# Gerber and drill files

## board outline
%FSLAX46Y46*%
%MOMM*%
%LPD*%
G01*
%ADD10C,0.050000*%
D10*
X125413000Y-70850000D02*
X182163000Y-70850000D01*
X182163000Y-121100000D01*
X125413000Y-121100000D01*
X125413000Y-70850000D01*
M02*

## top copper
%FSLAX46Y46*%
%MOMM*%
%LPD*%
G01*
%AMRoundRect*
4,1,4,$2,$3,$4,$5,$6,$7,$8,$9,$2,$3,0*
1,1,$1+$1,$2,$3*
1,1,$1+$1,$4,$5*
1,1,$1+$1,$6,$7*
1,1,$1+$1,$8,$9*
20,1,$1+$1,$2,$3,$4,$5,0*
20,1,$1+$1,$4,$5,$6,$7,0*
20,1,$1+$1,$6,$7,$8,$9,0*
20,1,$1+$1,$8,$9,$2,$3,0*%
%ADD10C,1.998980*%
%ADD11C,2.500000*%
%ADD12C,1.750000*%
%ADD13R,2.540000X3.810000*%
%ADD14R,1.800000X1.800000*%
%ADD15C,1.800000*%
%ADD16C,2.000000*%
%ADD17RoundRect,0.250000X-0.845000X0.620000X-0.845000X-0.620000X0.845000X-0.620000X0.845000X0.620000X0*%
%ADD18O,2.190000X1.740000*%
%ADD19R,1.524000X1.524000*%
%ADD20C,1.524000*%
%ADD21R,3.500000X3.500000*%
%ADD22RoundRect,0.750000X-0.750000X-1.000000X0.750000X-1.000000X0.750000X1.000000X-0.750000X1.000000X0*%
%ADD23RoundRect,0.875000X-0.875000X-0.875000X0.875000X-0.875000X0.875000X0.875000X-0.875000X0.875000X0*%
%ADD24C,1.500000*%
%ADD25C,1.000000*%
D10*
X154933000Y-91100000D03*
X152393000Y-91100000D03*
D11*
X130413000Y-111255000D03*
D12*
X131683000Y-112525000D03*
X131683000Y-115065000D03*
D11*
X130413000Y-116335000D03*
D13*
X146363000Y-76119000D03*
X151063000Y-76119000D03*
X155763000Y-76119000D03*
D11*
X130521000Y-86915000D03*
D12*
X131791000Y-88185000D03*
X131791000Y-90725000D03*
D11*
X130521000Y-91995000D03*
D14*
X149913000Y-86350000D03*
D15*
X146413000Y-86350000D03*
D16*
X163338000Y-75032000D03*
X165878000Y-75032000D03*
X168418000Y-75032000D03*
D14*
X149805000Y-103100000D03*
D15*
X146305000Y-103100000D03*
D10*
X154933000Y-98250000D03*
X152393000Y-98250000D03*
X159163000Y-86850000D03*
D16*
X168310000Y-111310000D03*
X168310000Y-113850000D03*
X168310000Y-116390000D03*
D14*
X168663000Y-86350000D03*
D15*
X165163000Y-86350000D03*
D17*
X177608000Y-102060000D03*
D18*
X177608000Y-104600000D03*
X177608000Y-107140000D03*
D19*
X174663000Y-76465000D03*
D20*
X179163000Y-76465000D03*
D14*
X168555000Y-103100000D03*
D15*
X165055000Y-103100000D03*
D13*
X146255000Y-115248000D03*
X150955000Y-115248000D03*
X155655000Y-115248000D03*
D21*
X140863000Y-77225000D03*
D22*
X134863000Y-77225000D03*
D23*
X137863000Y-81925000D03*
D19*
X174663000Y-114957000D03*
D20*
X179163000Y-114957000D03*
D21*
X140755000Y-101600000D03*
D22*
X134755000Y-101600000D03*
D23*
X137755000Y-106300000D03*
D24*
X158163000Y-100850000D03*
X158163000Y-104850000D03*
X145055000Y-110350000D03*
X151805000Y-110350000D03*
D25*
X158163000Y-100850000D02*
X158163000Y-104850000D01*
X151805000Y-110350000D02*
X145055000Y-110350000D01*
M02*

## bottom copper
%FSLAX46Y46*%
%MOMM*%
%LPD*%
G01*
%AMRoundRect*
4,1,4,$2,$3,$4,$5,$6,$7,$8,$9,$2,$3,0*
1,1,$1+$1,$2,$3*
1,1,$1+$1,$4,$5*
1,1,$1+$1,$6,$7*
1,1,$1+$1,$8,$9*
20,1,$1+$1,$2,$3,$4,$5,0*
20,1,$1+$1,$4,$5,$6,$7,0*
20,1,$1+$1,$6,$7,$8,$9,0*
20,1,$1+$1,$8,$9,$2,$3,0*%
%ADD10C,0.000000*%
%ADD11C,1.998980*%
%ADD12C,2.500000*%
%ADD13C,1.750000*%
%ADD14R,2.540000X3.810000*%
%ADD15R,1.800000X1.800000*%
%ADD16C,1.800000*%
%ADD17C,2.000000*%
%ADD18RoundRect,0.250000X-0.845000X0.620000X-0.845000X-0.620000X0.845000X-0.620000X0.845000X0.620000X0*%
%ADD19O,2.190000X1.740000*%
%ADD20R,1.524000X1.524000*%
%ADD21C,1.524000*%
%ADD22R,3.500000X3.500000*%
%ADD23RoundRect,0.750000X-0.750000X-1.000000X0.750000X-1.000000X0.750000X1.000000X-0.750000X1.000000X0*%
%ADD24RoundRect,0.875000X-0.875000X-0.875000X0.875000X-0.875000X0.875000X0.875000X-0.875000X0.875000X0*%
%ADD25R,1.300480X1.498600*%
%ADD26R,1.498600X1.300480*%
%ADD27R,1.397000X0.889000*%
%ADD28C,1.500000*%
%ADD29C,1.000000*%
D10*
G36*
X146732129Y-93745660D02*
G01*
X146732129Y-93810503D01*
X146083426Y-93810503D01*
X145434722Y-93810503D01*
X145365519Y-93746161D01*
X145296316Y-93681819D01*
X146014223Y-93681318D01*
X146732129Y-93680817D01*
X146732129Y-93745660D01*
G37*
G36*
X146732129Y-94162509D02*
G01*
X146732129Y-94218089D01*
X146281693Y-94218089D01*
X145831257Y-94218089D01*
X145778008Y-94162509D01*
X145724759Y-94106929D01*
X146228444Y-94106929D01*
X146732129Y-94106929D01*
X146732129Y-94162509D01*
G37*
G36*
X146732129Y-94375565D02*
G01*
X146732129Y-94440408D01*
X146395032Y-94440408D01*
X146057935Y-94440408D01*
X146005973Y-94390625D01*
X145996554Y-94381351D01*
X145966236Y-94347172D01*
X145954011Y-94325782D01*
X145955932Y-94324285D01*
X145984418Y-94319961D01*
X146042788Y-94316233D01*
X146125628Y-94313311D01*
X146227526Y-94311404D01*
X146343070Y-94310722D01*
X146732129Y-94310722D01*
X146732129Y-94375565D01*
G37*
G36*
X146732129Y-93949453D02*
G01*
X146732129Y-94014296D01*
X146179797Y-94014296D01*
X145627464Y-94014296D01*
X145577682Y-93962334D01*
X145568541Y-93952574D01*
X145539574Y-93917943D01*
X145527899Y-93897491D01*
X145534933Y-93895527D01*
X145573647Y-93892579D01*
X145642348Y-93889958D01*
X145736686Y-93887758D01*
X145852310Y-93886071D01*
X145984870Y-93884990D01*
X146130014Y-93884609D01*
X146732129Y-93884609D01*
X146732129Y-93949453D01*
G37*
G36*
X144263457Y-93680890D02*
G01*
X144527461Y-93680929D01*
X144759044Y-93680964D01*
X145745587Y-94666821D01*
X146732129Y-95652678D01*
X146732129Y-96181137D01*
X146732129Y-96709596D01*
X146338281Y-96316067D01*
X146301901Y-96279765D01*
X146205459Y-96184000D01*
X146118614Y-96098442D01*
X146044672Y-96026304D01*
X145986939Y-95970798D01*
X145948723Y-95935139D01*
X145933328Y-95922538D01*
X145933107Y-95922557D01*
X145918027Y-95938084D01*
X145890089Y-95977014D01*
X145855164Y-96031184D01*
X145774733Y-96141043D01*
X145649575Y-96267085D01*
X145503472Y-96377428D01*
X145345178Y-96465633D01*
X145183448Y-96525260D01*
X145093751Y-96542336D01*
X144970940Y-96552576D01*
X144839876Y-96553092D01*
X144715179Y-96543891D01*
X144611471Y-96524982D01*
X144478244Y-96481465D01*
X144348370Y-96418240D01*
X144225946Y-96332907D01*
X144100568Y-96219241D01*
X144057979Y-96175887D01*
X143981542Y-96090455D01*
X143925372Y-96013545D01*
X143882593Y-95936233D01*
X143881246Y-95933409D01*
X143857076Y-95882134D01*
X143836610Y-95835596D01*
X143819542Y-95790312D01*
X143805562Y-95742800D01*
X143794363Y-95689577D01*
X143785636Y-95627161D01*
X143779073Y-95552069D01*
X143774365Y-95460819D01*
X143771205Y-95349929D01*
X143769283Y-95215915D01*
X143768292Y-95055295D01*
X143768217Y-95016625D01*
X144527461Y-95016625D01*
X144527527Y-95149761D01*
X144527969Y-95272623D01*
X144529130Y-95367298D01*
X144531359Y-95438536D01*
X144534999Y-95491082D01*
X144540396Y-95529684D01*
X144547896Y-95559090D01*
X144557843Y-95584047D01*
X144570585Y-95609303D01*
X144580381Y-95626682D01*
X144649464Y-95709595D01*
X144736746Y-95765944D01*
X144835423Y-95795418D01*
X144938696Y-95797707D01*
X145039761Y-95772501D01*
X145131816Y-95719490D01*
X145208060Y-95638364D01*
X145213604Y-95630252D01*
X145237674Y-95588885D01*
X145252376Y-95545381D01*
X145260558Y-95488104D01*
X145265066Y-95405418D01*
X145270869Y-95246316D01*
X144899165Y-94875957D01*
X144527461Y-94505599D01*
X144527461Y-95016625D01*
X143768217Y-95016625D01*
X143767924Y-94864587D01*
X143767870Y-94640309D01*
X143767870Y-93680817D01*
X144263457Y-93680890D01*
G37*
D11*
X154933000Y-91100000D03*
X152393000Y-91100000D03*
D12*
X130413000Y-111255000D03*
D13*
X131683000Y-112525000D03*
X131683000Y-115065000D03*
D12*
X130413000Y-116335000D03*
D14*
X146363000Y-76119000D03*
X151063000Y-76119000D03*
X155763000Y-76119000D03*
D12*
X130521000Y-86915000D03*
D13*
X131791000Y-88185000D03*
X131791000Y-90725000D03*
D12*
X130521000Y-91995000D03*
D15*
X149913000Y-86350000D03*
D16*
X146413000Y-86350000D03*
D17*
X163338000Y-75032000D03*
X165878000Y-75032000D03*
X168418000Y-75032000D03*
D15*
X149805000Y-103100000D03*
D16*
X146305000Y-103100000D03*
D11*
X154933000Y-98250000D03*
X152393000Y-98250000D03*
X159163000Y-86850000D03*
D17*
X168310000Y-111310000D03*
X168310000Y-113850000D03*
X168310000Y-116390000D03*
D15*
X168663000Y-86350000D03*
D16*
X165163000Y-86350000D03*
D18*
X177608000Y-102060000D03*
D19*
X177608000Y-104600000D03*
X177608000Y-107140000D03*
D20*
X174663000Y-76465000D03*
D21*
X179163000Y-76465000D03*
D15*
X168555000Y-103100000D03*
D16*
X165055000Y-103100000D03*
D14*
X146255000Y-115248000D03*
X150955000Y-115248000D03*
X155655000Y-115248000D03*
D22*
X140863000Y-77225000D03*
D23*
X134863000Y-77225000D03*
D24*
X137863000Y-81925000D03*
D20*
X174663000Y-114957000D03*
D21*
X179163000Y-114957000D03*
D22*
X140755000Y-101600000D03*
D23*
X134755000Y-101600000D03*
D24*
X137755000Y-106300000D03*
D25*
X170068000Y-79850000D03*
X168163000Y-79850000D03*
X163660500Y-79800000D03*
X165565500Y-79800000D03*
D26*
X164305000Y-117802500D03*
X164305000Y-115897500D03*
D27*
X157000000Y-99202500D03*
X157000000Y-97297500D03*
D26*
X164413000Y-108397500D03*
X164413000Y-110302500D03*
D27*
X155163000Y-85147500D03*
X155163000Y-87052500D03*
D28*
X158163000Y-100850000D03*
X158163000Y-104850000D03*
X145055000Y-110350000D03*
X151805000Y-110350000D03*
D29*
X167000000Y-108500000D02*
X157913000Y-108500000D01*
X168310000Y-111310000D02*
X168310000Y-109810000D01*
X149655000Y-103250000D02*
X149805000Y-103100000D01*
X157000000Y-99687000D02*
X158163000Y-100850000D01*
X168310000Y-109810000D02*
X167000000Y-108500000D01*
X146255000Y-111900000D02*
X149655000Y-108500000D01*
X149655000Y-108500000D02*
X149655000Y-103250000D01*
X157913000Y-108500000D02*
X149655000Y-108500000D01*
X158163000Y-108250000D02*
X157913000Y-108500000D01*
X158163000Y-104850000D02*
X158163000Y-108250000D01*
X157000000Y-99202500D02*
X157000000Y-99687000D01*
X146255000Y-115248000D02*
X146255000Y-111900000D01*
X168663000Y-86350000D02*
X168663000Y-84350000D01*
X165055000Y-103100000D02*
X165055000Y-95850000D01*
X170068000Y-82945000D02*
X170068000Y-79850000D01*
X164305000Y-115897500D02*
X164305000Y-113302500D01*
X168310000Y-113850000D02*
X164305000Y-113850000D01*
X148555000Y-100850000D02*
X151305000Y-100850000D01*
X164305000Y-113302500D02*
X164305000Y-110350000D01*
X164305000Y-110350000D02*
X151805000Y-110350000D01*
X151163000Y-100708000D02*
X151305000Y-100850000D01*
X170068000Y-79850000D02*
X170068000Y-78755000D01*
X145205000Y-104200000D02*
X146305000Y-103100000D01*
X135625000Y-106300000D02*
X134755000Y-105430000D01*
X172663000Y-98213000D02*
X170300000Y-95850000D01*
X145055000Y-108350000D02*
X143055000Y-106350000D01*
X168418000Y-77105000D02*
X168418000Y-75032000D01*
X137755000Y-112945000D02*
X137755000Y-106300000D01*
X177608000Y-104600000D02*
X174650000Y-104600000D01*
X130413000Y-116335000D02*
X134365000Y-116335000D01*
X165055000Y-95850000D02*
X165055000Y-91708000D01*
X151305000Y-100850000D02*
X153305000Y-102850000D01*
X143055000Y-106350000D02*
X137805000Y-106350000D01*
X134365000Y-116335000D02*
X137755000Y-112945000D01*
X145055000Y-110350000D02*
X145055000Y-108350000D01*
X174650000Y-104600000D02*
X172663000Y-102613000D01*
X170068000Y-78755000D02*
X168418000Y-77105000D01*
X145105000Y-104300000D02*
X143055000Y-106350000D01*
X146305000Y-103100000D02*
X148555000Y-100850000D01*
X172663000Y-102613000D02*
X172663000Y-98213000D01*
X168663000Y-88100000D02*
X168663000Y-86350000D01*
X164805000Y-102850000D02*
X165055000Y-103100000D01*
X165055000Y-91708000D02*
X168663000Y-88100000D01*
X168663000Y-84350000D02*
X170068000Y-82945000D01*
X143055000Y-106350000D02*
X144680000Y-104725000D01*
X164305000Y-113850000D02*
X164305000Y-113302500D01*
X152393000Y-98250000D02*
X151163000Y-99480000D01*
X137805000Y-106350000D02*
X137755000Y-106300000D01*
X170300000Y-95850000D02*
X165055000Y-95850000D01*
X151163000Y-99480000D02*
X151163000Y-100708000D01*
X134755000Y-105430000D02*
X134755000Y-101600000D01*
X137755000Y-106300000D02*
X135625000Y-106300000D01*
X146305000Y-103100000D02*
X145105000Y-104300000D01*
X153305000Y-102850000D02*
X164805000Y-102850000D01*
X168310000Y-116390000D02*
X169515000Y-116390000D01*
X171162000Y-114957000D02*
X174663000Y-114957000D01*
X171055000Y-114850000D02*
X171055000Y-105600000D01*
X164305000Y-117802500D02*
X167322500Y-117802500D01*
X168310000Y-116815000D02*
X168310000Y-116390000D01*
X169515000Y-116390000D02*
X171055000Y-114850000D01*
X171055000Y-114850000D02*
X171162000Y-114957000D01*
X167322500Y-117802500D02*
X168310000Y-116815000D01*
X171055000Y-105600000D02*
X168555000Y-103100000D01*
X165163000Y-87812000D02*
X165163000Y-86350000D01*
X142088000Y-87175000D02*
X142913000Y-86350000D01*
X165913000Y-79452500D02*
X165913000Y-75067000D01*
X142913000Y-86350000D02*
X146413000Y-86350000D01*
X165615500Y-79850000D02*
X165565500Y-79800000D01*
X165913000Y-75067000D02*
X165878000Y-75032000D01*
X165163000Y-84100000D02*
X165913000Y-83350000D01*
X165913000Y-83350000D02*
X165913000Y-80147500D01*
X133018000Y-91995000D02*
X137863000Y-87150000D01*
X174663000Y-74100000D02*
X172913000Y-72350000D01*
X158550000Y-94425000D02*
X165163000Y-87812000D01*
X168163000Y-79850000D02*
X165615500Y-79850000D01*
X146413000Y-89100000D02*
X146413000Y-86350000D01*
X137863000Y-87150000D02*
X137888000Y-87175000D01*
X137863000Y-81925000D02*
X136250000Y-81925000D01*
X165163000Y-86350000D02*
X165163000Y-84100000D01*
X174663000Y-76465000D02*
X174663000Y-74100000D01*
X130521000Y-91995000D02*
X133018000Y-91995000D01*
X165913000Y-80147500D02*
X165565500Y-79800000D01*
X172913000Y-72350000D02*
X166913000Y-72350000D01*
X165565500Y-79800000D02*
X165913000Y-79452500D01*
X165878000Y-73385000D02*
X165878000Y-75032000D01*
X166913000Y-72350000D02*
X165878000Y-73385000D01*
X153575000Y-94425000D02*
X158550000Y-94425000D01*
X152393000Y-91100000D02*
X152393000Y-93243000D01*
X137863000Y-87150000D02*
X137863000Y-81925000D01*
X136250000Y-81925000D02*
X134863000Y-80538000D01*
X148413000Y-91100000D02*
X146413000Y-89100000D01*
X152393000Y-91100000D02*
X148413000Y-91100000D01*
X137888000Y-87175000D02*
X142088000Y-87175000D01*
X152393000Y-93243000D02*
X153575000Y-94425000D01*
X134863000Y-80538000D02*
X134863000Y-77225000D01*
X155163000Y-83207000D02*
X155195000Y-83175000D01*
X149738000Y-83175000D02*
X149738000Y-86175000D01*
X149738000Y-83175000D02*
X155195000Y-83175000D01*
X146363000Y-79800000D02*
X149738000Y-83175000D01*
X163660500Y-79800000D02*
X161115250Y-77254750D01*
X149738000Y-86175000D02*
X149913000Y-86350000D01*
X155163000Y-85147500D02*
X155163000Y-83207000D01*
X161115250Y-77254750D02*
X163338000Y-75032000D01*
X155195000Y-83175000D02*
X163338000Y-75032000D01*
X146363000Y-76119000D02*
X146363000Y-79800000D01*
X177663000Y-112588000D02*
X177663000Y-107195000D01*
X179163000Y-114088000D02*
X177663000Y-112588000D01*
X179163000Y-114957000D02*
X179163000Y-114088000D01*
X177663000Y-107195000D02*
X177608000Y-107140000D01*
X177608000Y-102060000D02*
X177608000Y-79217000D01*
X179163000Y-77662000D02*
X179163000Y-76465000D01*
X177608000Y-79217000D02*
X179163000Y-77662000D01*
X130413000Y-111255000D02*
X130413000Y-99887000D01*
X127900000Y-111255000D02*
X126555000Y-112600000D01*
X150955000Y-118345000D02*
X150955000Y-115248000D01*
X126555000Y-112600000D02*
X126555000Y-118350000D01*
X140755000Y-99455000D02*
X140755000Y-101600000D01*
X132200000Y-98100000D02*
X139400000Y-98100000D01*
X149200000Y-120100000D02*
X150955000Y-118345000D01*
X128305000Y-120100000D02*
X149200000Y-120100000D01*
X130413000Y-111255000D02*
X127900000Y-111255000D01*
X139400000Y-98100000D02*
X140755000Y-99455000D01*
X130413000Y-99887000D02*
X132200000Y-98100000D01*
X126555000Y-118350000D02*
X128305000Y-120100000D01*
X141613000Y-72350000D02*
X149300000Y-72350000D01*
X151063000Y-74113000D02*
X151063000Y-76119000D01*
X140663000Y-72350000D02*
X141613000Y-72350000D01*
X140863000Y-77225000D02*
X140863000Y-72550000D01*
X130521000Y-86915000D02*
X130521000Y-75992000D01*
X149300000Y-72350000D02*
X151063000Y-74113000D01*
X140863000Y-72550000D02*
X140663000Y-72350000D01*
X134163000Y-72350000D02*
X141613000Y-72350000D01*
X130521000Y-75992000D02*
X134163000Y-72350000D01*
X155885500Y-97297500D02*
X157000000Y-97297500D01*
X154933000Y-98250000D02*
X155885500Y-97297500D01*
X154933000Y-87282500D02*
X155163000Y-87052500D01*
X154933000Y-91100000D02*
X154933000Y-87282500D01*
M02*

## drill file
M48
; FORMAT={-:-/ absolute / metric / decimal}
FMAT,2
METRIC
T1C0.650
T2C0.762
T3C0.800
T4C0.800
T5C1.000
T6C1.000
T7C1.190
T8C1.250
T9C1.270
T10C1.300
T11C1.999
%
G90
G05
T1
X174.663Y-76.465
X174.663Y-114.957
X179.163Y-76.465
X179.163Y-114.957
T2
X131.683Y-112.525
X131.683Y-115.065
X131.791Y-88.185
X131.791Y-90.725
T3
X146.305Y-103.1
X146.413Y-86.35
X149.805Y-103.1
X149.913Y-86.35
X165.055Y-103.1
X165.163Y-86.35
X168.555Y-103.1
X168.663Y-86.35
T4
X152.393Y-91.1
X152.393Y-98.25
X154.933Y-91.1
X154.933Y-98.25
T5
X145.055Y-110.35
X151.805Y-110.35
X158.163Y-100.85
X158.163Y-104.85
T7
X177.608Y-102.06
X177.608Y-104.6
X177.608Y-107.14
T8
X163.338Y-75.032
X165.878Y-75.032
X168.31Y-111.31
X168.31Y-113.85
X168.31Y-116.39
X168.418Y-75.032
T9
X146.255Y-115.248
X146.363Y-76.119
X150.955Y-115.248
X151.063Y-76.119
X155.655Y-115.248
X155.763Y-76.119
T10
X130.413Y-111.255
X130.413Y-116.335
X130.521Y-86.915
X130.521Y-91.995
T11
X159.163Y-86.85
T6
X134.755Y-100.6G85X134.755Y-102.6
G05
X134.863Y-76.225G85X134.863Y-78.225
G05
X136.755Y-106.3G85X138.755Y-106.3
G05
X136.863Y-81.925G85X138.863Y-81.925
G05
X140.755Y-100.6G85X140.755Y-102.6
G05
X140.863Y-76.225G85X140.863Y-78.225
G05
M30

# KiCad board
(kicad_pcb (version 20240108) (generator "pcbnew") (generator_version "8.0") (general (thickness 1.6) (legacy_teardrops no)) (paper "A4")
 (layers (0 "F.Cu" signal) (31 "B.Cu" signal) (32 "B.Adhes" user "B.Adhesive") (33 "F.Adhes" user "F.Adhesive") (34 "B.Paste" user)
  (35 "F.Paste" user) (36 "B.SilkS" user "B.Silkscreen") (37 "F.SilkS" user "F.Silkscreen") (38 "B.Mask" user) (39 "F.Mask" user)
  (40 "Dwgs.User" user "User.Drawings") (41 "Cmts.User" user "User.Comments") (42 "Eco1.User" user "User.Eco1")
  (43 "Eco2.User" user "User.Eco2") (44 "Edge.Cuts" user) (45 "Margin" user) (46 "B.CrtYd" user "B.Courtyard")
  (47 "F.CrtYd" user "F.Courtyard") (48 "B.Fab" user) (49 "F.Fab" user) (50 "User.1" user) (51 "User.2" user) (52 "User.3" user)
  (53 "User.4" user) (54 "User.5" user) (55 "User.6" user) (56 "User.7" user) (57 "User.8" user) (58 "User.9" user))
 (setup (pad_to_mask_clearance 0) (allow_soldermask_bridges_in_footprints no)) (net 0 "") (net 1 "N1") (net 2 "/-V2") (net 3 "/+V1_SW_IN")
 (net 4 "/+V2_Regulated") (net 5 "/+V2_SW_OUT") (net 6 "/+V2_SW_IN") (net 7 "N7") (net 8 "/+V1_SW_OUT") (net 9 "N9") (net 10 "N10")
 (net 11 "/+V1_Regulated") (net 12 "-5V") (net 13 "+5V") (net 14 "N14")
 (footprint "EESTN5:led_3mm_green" (layer "F.Cu") (at 153.663 91.1 -90)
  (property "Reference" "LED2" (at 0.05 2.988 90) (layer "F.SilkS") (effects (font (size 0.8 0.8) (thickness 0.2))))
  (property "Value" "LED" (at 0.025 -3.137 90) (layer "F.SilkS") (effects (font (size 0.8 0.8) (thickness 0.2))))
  (pad "1" thru_hole circle (at 0 -1.27 270) (size 1.99898 1.99898) (drill 0.8001) (layers "*.Cu" "*.Mask" "F.SilkS")
   (remove_unused_layers no) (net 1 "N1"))
  (pad "2" thru_hole circle (at 0 1.27 270) (size 1.99898 1.99898) (drill 0.8001) (layers "*.Cu" "*.Mask" "F.SilkS")
   (remove_unused_layers no) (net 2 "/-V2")))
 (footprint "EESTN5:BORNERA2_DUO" (layer "F.Cu") (at 130.413 113.795 -90)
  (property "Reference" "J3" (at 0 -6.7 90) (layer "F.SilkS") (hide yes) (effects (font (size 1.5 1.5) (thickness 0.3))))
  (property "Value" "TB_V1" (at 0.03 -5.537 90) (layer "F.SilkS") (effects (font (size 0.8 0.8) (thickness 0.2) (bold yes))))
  (pad "1" thru_hole circle (at -2.54 0 270) (size 2.5 2.5) (drill 1.3) (layers "*.Cu" "*.Mask" "F.SilkS") (remove_unused_layers no)
   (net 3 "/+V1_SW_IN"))
  (pad "1" thru_hole circle (at -1.27 -1.27 270) (size 1.75 1.75) (drill 0.762) (layers "*.Cu" "*.Mask") (remove_unused_layers no)
   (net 3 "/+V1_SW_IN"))
  (pad "2" thru_hole circle (at 1.27 -1.27 270) (size 1.75 1.75) (drill 0.762) (layers "*.Cu" "*.Mask") (remove_unused_layers no)
   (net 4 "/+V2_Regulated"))
  (pad "2" thru_hole circle (at 2.54 0 270) (size 2.5 2.5) (drill 1.3) (layers "*.Cu" "*.Mask" "F.SilkS") (remove_unused_layers no)
   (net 4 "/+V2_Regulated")))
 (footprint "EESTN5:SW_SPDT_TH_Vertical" (layer "F.Cu") (at 151.063 76.119 90)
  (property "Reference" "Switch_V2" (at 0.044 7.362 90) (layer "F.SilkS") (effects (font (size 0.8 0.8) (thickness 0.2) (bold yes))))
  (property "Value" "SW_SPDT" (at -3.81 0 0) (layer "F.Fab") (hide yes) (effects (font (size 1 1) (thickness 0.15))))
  (pad "1" thru_hole rect (at 0 -4.7 90) (size 3.81 2.54) (drill 1.27) (layers "*.Cu" "*.Mask") (remove_unused_layers no)
   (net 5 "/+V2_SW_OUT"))
  (pad "2" thru_hole rect (at 0 0 90) (size 3.81 2.54) (drill 1.27) (layers "*.Cu" "*.Mask") (remove_unused_layers no) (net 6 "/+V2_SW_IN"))
  (pad "3" thru_hole rect (at 0 4.7 90) (size 3.81 2.54) (drill 1.27) (layers "*.Cu" "*.Mask") (remove_unused_layers no) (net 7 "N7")))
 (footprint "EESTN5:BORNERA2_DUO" (layer "F.Cu") (at 130.521 89.455 -90)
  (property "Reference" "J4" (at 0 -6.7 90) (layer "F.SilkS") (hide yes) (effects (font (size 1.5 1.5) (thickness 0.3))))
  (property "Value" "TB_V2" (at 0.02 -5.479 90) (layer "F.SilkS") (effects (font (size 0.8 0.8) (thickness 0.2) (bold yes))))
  (pad "1" thru_hole circle (at -2.54 0 270) (size 2.5 2.5) (drill 1.3) (layers "*.Cu" "*.Mask" "F.SilkS") (remove_unused_layers no)
   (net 6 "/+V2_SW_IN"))
  (pad "1" thru_hole circle (at -1.27 -1.27 270) (size 1.75 1.75) (drill 0.762) (layers "*.Cu" "*.Mask") (remove_unused_layers no)
   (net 6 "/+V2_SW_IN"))
  (pad "2" thru_hole circle (at 1.27 -1.27 270) (size 1.75 1.75) (drill 0.762) (layers "*.Cu" "*.Mask") (remove_unused_layers no)
   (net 2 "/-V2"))
  (pad "2" thru_hole circle (at 2.54 0 270) (size 2.5 2.5) (drill 1.3) (layers "*.Cu" "*.Mask" "F.SilkS") (remove_unused_layers no)
   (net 2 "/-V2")))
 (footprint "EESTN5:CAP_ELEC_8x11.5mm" (layer "F.Cu") (at 148.163 86.35 90)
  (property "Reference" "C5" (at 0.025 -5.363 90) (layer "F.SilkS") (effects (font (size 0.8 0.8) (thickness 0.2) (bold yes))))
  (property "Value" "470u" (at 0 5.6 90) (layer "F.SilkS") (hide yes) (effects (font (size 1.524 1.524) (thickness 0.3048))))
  (pad "1" thru_hole rect (at 0 1.75 90) (size 1.8 1.8) (drill 0.8) (layers "*.Cu" "*.Mask" "F.SilkS") (remove_unused_layers no)
   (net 5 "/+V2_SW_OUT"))
  (pad "2" thru_hole circle (at 0 -1.75 90) (size 1.8 1.8) (drill 0.8) (layers "*.Cu" "*.Mask" "F.SilkS") (remove_unused_layers no)
   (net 2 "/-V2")))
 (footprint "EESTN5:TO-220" (layer "F.Cu") (at 165.878 75.032)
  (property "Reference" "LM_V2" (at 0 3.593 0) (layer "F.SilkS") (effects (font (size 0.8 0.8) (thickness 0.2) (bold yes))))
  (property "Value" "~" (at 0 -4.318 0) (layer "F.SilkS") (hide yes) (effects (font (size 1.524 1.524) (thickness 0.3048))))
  (pad "1" thru_hole circle (at -2.54 0) (size 2 2) (drill 1.24968) (layers "*.Cu" "*.Mask" "F.SilkS") (remove_unused_layers no)
   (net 5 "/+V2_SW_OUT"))
  (pad "2" thru_hole circle (at 0 0) (size 2 2) (drill 1.24968) (layers "*.Cu" "*.Mask" "F.SilkS") (remove_unused_layers no) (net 2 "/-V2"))
  (pad "3" thru_hole circle (at 2.54 0) (size 2 2) (drill 1.24968) (layers "*.Cu" "*.Mask" "F.SilkS") (remove_unused_layers no)
   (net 4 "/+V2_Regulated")))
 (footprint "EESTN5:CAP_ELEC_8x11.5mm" (layer "F.Cu") (at 148.055 103.1 90)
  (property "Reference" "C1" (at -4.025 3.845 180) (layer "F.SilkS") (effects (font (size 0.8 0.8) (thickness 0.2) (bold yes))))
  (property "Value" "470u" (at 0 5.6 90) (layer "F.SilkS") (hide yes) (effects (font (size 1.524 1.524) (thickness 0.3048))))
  (pad "1" thru_hole rect (at 0 1.75 90) (size 1.8 1.8) (drill 0.8) (layers "*.Cu" "*.Mask" "F.SilkS") (remove_unused_layers no)
   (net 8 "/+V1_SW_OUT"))
  (pad "2" thru_hole circle (at 0 -1.75 90) (size 1.8 1.8) (drill 0.8) (layers "*.Cu" "*.Mask" "F.SilkS") (remove_unused_layers no)
   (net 4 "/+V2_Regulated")))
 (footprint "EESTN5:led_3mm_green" (layer "F.Cu") (at 153.663 98.25 -90)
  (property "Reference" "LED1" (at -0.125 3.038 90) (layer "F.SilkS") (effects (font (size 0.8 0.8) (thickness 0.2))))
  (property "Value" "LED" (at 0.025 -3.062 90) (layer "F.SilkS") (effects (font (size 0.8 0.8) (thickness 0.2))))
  (pad "1" thru_hole circle (at 0 -1.27 270) (size 1.99898 1.99898) (drill 0.8001) (layers "*.Cu" "*.Mask" "F.SilkS")
   (remove_unused_layers no) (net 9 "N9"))
  (pad "2" thru_hole circle (at 0 1.27 270) (size 1.99898 1.99898) (drill 0.8001) (layers "*.Cu" "*.Mask" "F.SilkS")
   (remove_unused_layers no) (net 4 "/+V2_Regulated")))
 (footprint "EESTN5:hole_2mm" (layer "F.Cu") (at 159.163 86.85)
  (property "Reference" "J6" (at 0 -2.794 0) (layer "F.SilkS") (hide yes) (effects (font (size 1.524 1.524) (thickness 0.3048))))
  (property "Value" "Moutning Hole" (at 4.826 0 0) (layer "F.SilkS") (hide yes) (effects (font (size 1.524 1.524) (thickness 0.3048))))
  (pad "1" thru_hole circle (at 0 0) (size 1.99898 1.99898) (drill 1.99898) (layers "*.Cu" "F.SilkS") (remove_unused_layers no)
   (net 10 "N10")))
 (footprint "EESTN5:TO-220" (layer "F.Cu") (at 168.31 113.85 -90)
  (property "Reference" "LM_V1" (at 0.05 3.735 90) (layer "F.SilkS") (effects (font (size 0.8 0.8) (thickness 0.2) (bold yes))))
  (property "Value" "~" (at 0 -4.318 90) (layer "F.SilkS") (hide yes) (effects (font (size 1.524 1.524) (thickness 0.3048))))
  (pad "1" thru_hole circle (at -2.54 0 270) (size 2 2) (drill 1.24968) (layers "*.Cu" "*.Mask" "F.SilkS") (remove_unused_layers no)
   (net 8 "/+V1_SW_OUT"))
  (pad "2" thru_hole circle (at 0 0 270) (size 2 2) (drill 1.24968) (layers "*.Cu" "*.Mask" "F.SilkS") (remove_unused_layers no)
   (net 4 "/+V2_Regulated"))
  (pad "3" thru_hole circle (at 2.54 0 270) (size 2 2) (drill 1.24968) (layers "*.Cu" "*.Mask" "F.SilkS") (remove_unused_layers no)
   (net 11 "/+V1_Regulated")))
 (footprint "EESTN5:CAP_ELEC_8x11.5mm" (layer "F.Cu") (at 166.913 86.35 90)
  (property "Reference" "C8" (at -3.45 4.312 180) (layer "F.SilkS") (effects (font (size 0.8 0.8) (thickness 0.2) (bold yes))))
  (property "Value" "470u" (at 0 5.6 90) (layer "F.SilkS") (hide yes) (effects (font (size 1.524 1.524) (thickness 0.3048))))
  (pad "1" thru_hole rect (at 0 1.75 90) (size 1.8 1.8) (drill 0.8) (layers "*.Cu" "*.Mask" "F.SilkS") (remove_unused_layers no)
   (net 4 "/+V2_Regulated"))
  (pad "2" thru_hole circle (at 0 -1.75 90) (size 1.8 1.8) (drill 0.8) (layers "*.Cu" "*.Mask" "F.SilkS") (remove_unused_layers no)
   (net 2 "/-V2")))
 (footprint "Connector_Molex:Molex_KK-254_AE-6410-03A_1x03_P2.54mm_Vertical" (layer "F.Cu") (at 177.608 102.06 -90)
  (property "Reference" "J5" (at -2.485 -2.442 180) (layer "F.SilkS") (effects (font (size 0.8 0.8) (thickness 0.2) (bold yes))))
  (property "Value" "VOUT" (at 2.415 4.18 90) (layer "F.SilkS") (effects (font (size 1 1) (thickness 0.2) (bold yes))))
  (pad "1" thru_hole roundrect (at 0 0 270) (size 1.74 2.19) (drill 1.19) (layers "*.Cu" "*.Mask") (remove_unused_layers no)
   (roundrect_rratio 0.143678) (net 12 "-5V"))
  (pad "2" thru_hole oval (at 2.54 0 270) (size 1.74 2.19) (drill 1.19) (layers "*.Cu" "*.Mask") (remove_unused_layers no)
   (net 4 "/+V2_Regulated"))
  (pad "3" thru_hole oval (at 5.08 0 270) (size 1.74 2.19) (drill 1.19) (layers "*.Cu" "*.Mask") (remove_unused_layers no) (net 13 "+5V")))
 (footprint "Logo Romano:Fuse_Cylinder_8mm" (layer "F.Cu") (at 176.913 76.465 -90)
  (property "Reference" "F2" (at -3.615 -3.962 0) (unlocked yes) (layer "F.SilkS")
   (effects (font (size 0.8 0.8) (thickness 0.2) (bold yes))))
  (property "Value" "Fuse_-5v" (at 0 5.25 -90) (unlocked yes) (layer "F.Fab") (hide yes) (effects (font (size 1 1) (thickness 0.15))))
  (pad "1" thru_hole rect (at 0 2.25 270) (size 1.524 1.524) (drill 0.65) (layers "*.Cu" "*.Mask" "F.SilkS") (remove_unused_layers no)
   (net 2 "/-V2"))
  (pad "2" thru_hole circle (at 0 -2.25 270) (size 1.524 1.524) (drill 0.65) (layers "*.Cu" "*.Mask" "F.SilkS") (remove_unused_layers no)
   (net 12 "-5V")))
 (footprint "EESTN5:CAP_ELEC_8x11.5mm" (layer "F.Cu") (at 166.805 103.1 90)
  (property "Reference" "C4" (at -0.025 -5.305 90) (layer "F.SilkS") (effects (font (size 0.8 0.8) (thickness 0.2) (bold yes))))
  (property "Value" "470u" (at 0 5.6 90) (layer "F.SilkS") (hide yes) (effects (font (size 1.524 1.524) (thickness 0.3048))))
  (pad "1" thru_hole rect (at 0 1.75 90) (size 1.8 1.8) (drill 0.8) (layers "*.Cu" "*.Mask" "F.SilkS") (remove_unused_layers no)
   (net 11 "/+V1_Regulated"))
  (pad "2" thru_hole circle (at 0 -1.75 90) (size 1.8 1.8) (drill 0.8) (layers "*.Cu" "*.Mask" "F.SilkS") (remove_unused_layers no)
   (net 4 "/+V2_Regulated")))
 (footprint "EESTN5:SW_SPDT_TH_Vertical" (layer "F.Cu") (at 150.955 115.248 90)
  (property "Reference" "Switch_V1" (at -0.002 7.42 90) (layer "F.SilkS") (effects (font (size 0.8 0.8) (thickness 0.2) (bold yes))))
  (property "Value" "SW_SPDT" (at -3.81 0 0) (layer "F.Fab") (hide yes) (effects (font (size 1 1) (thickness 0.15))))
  (pad "1" thru_hole rect (at 0 -4.7 90) (size 3.81 2.54) (drill 1.27) (layers "*.Cu" "*.Mask") (remove_unused_layers no)
   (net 8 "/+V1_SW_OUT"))
  (pad "2" thru_hole rect (at 0 0 90) (size 3.81 2.54) (drill 1.27) (layers "*.Cu" "*.Mask") (remove_unused_layers no) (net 3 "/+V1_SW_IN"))
  (pad "3" thru_hole rect (at 0 4.7 90) (size 3.81 2.54) (drill 1.27) (layers "*.Cu" "*.Mask") (remove_unused_layers no) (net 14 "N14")))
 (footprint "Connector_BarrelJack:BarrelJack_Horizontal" (layer "F.Cu") (at 140.863 77.225)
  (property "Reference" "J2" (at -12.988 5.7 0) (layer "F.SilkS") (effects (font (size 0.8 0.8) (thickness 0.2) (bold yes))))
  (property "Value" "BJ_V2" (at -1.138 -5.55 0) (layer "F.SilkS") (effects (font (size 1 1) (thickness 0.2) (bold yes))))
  (pad "1" thru_hole rect (at 0 0) (size 3.5 3.5) (drill oval 1 3) (layers "*.Cu" "*.Mask") (remove_unused_layers no) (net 6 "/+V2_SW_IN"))
  (pad "2" thru_hole roundrect (at -6 0) (size 3 3.5) (drill oval 1 3) (layers "*.Cu" "*.Mask") (remove_unused_layers no)
   (roundrect_rratio 0.25) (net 2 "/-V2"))
  (pad "3" thru_hole roundrect (at -3 4.7) (size 3.5 3.5) (drill oval 3 1) (layers "*.Cu" "*.Mask") (remove_unused_layers no)
   (roundrect_rratio 0.25) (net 2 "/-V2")))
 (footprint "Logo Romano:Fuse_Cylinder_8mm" (layer "F.Cu") (at 176.913 114.957 -90)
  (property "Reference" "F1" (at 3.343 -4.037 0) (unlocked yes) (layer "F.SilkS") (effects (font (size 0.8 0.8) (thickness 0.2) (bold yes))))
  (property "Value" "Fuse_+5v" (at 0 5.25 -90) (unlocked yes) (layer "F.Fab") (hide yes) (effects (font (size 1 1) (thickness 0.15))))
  (pad "1" thru_hole rect (at 0 2.25 270) (size 1.524 1.524) (drill 0.65) (layers "*.Cu" "*.Mask" "F.SilkS") (remove_unused_layers no)
   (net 11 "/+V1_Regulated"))
  (pad "2" thru_hole circle (at 0 -2.25 270) (size 1.524 1.524) (drill 0.65) (layers "*.Cu" "*.Mask" "F.SilkS") (remove_unused_layers no)
   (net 13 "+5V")))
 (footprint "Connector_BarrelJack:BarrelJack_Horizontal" (layer "F.Cu") (at 140.755 101.6)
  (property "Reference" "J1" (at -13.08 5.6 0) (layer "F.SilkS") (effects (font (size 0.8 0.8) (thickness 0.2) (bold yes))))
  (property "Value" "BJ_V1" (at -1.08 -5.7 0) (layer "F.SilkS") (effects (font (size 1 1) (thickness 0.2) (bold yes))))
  (pad "1" thru_hole rect (at 0 0) (size 3.5 3.5) (drill oval 1 3) (layers "*.Cu" "*.Mask") (remove_unused_layers no) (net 3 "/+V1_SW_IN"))
  (pad "2" thru_hole roundrect (at -6 0) (size 3 3.5) (drill oval 1 3) (layers "*.Cu" "*.Mask") (remove_unused_layers no)
   (roundrect_rratio 0.25) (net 4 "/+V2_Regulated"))
  (pad "3" thru_hole roundrect (at -3 4.7) (size 3.5 3.5) (drill oval 3 1) (layers "*.Cu" "*.Mask") (remove_unused_layers no)
   (roundrect_rratio 0.25) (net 4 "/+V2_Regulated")))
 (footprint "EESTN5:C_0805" (layer "B.Cu") (at 169.1155 79.85)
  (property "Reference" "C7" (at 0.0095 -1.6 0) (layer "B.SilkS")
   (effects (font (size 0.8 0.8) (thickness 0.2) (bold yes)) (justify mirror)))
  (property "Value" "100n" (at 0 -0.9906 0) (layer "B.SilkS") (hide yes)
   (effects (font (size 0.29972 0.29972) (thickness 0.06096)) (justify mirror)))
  (pad "1" smd rect (at 0.9525 0) (size 1.30048 1.4986) (layers "B.Cu" "B.Paste" "B.Mask") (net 4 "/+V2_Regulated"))
  (pad "2" smd rect (at -0.9525 0) (size 1.30048 1.4986) (layers "B.Cu" "B.Paste" "B.Mask") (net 2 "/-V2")))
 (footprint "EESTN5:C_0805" (layer "B.Cu") (at 164.613 79.8 180)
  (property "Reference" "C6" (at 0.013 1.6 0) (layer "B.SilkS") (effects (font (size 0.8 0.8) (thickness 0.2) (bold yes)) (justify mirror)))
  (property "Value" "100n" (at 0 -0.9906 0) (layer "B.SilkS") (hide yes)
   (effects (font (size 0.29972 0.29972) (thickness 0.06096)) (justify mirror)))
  (pad "1" smd rect (at 0.9525 0 180) (size 1.30048 1.4986) (layers "B.Cu" "B.Paste" "B.Mask") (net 5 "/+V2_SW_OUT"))
  (pad "2" smd rect (at -0.9525 0 180) (size 1.30048 1.4986) (layers "B.Cu" "B.Paste" "B.Mask") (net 2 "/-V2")))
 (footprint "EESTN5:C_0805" (layer "B.Cu") (at 164.305 116.85 -90)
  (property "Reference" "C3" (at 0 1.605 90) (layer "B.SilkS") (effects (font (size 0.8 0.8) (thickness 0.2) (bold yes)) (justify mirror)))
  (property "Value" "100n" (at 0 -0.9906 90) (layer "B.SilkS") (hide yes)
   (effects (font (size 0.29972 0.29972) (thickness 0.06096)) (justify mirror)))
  (pad "1" smd rect (at 0.9525 0 270) (size 1.30048 1.4986) (layers "B.Cu" "B.Paste" "B.Mask") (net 11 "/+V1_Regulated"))
  (pad "2" smd rect (at -0.9525 0 270) (size 1.30048 1.4986) (layers "B.Cu" "B.Paste" "B.Mask") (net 4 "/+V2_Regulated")))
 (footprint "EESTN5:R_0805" (layer "B.Cu") (at 157 98.25 90)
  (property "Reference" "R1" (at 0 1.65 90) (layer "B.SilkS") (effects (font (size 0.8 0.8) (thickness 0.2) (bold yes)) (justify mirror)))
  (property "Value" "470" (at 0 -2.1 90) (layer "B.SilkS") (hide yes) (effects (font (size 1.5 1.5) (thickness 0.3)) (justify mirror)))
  (pad "1" smd rect (at -0.9525 0 90) (size 0.889 1.397) (layers "B.Cu" "B.Paste" "B.Mask") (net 8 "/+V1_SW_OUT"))
  (pad "2" smd rect (at 0.9525 0 90) (size 0.889 1.397) (layers "B.Cu" "B.Paste" "B.Mask") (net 9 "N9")))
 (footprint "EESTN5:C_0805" (layer "B.Cu") (at 164.413 109.35 90)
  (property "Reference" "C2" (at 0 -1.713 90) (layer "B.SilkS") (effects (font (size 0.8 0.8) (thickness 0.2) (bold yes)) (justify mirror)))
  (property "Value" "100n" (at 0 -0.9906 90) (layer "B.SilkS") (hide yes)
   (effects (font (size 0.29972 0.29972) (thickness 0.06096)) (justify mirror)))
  (pad "1" smd rect (at 0.9525 0 90) (size 1.30048 1.4986) (layers "B.Cu" "B.Paste" "B.Mask") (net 8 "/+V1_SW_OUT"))
  (pad "2" smd rect (at -0.9525 0 90) (size 1.30048 1.4986) (layers "B.Cu" "B.Paste" "B.Mask") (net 4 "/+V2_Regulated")))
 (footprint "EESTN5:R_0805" (layer "B.Cu") (at 155.163 86.1 -90)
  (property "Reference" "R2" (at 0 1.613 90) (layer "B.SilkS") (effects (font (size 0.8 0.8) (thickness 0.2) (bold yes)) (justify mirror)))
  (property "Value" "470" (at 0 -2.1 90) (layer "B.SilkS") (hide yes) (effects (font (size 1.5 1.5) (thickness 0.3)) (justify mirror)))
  (pad "1" smd rect (at -0.9525 0 270) (size 0.889 1.397) (layers "B.Cu" "B.Paste" "B.Mask") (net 5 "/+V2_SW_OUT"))
  (pad "2" smd rect (at 0.9525 0 270) (size 0.889 1.397) (layers "B.Cu" "B.Paste" "B.Mask") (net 1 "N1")))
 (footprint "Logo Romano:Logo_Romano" (layer "B.Cu") (at 145.25 95.2 -90)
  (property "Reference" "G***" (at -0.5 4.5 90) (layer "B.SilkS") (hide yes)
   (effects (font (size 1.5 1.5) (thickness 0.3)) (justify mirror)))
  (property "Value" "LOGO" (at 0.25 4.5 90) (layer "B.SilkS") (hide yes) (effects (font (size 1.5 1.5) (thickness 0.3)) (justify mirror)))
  (fp_poly
   (pts (xy -1.453839 -0.115519) (xy -1.389497 -0.184722) (xy -1.389497 -0.833426) (xy -1.389497 -1.482129) (xy -1.45434 -1.482129)
    (xy -1.519183 -1.482129) (xy -1.518682 -0.764223) (xy -1.518181 -0.046316))
   (stroke (width 0) (type solid)) (fill solid) (layer "B.Cu"))
  (fp_poly
   (pts (xy -1.037491 -0.528008) (xy -0.981911 -0.581257) (xy -0.981911 -1.031693) (xy -0.981911 -1.482129) (xy -1.037491 -1.482129)
    (xy -1.093071 -1.482129) (xy -1.093071 -0.978444) (xy -1.093071 -0.474759))
   (stroke (width 0) (type solid)) (fill solid) (layer "B.Cu"))
  (fp_poly
   (pts (xy -0.852828 -0.716236) (xy -0.818649 -0.746554) (xy -0.809375 -0.755973) (xy -0.759592 -0.807935) (xy -0.759592 -1.145032)
    (xy -0.759592 -1.482129) (xy -0.824435 -1.482129) (xy -0.889278 -1.482129) (xy -0.889278 -1.09307) (xy -0.888596 -0.977526)
    (xy -0.886689 -0.875628) (xy -0.883767 -0.792788) (xy -0.880039 -0.734418) (xy -0.875715 -0.705932) (xy -0.874218 -0.704011))
   (stroke (width 0) (type solid)) (fill solid) (layer "B.Cu"))
  (fp_poly
   (pts (xy -1.282057 -0.289574) (xy -1.247426 -0.318541) (xy -1.237666 -0.327682) (xy -1.185704 -0.377464) (xy -1.185704 -0.929797)
    (xy -1.185704 -1.482129) (xy -1.250547 -1.482129) (xy -1.315391 -1.482129) (xy -1.315391 -0.880014) (xy -1.31501 -0.73487)
    (xy -1.313929 -0.60231) (xy -1.312242 -0.486686) (xy -1.310042 -0.392348) (xy -1.307421 -0.323647) (xy -1.304473 -0.284933)
    (xy -1.302509 -0.277899))
   (stroke (width 0) (type solid)) (fill solid) (layer "B.Cu"))
  (fp_poly
   (pts (xy -0.335413 1.482076) (xy -0.144705 1.481708) (xy 0.015915 1.480717) (xy 0.149929 1.478795) (xy 0.260819 1.475635)
    (xy 0.352069 1.470927) (xy 0.427161 1.464364) (xy 0.489577 1.455637) (xy 0.5428 1.444438) (xy 0.590312 1.430458) (xy 0.635596 1.41339)
    (xy 0.682134 1.392924) (xy 0.733409 1.368754) (xy 0.736233 1.367407) (xy 0.813545 1.324628) (xy 0.890455 1.268458)
    (xy 0.975887 1.192021) (xy 1.019241 1.149432) (xy 1.132907 1.024054) (xy 1.21824 0.90163) (xy 1.281465 0.771756) (xy 1.324982 0.638529)
    (xy 1.343891 0.534821) (xy 1.353092 0.410124) (xy 1.352576 0.27906) (xy 1.342336 0.156249) (xy 1.32526 0.066552) (xy 1.265633 -0.095178)
    (xy 1.177428 -0.253472) (xy 1.067085 -0.399575) (xy 0.941043 -0.524733) (xy 0.831184 -0.605164) (xy 0.777014 -0.640089)
    (xy 0.738084 -0.668027) (xy 0.722557 -0.683107) (xy 0.722538 -0.683328) (xy 0.735139 -0.698723) (xy 0.770798 -0.736939)
    (xy 0.826304 -0.794672) (xy 0.898442 -0.868614) (xy 0.984 -0.955459) (xy 1.079765 -1.051901) (xy 1.116067 -1.088281)
    (xy 1.509596 -1.482129) (xy 0.981137 -1.482129) (xy 0.452678 -1.482129) (xy -0.533179 -0.495587) (xy -1.519036 0.490956)
    (xy -1.519071 0.722539) (xy -0.694401 0.722539) (xy -0.324043 0.350835) (xy 0.046316 -0.020869) (xy 0.205418 -0.015066)
    (xy 0.288104 -0.010558) (xy 0.345381 -0.002376) (xy 0.388885 0.012326) (xy 0.430252 0.036396) (xy 0.438364 0.04194)
    (xy 0.51949 0.118184) (xy 0.572501 0.210239) (xy 0.597707 0.311304) (xy 0.595418 0.414577) (xy 0.565944 0.513254) (xy 0.509595 0.600536)
    (xy 0.426682 0.669619) (xy 0.409303 0.679415) (xy 0.384047 0.692157) (xy 0.35909 0.702104) (xy 0.329684 0.709604) (xy 0.291082 0.715001)
    (xy 0.238536 0.718641) (xy 0.167298 0.72087) (xy 0.072623 0.722031) (xy -0.050239 0.722473) (xy -0.183375 0.722539)
    (xy -0.694401 0.722539) (xy -1.519071 0.722539) (xy -1.51911 0.986543) (xy -1.519183 1.48213) (xy -0.559691 1.48213))
   (stroke (width 0) (type solid)) (fill solid) (layer "B.Cu")))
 (gr_rect (start 125.413 70.85) (end 182.163 121.1) (stroke (width 0.05) (type default)) (fill none) (layer "Edge.Cuts"))
 (segment (start 158.163 100.85) (end 158.163 104.85) (width 1) (layer "F.Cu") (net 8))
 (via (at 158.163 100.85) (size 1.5) (drill 1) (layers "F.Cu" "B.Cu") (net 8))
 (via (at 158.163 104.85) (size 1.5) (drill 1) (layers "F.Cu" "B.Cu") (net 8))
 (segment (start 167 108.5) (end 157.913 108.5) (width 1) (layer "B.Cu") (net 8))
 (segment (start 168.31 111.31) (end 168.31 109.81) (width 1) (layer "B.Cu") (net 8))
 (segment (start 149.655 103.25) (end 149.805 103.1) (width 1) (layer "B.Cu") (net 8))
 (segment (start 157 99.687) (end 158.163 100.85) (width 1) (layer "B.Cu") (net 8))
 (segment (start 168.31 109.81) (end 167 108.5) (width 1) (layer "B.Cu") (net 8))
 (segment (start 146.255 111.9) (end 149.655 108.5) (width 1) (layer "B.Cu") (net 8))
 (segment (start 149.655 108.5) (end 149.655 103.25) (width 1) (layer "B.Cu") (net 8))
 (segment (start 157.913 108.5) (end 149.655 108.5) (width 1) (layer "B.Cu") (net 8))
 (segment (start 158.163 108.25) (end 157.913 108.5) (width 1) (layer "B.Cu") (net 8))
 (segment (start 158.163 104.85) (end 158.163 108.25) (width 1) (layer "B.Cu") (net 8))
 (segment (start 157 99.2025) (end 157 99.687) (width 1) (layer "B.Cu") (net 8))
 (segment (start 146.255 115.248) (end 146.255 111.9) (width 1) (layer "B.Cu") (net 8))
 (segment (start 151.805 110.35) (end 145.055 110.35) (width 1) (layer "F.Cu") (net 4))
 (via (at 145.055 110.35) (size 1.5) (drill 1) (layers "F.Cu" "B.Cu") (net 4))
 (via (at 151.805 110.35) (size 1.5) (drill 1) (layers "F.Cu" "B.Cu") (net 4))
 (segment (start 168.663 86.35) (end 168.663 84.35) (width 1) (layer "B.Cu") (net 4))
 (segment (start 165.055 103.1) (end 165.055 95.85) (width 1) (layer "B.Cu") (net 4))
 (segment (start 170.068 82.945) (end 170.068 79.85) (width 1) (layer "B.Cu") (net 4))
 (segment (start 164.305 115.8975) (end 164.305 113.3025) (width 1) (layer "B.Cu") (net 4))
 (segment (start 168.31 113.85) (end 164.305 113.85) (width 1) (layer "B.Cu") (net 4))
 (segment (start 148.555 100.85) (end 151.305 100.85) (width 1) (layer "B.Cu") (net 4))
 (segment (start 164.305 113.3025) (end 164.305 110.35) (width 1) (layer "B.Cu") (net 4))
 (segment (start 164.305 110.35) (end 151.805 110.35) (width 1) (layer "B.Cu") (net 4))
 (segment (start 151.163 100.708) (end 151.305 100.85) (width 1) (layer "B.Cu") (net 4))
 (segment (start 170.068 79.85) (end 170.068 78.755) (width 1) (layer "B.Cu") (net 4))
 (segment (start 145.205 104.2) (end 146.305 103.1) (width 1) (layer "B.Cu") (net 4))
 (segment (start 135.625 106.3) (end 134.755 105.43) (width 1) (layer "B.Cu") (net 4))
 (segment (start 172.663 98.213) (end 170.3 95.85) (width 1) (layer "B.Cu") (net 4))
 (segment (start 145.055 108.35) (end 143.055 106.35) (width 1) (layer "B.Cu") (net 4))
 (segment (start 168.418 77.105) (end 168.418 75.032) (width 1) (layer "B.Cu") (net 4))
 (segment (start 137.755 112.945) (end 137.755 106.3) (width 1) (layer "B.Cu") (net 4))
 (segment (start 177.608 104.6) (end 174.65 104.6) (width 1) (layer "B.Cu") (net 4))
 (segment (start 130.413 116.335) (end 134.365 116.335) (width 1) (layer "B.Cu") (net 4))
 (segment (start 165.055 95.85) (end 165.055 91.708) (width 1) (layer "B.Cu") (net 4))
 (segment (start 151.305 100.85) (end 153.305 102.85) (width 1) (layer "B.Cu") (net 4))
 (segment (start 143.055 106.35) (end 137.805 106.35) (width 1) (layer "B.Cu") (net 4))
 (segment (start 134.365 116.335) (end 137.755 112.945) (width 1) (layer "B.Cu") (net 4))
 (segment (start 145.055 110.35) (end 145.055 108.35) (width 1) (layer "B.Cu") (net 4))
 (segment (start 174.65 104.6) (end 172.663 102.613) (width 1) (layer "B.Cu") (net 4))
 (segment (start 170.068 78.755) (end 168.418 77.105) (width 1) (layer "B.Cu") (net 4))
 (segment (start 145.105 104.3) (end 143.055 106.35) (width 1) (layer "B.Cu") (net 4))
 (segment (start 146.305 103.1) (end 148.555 100.85) (width 1) (layer "B.Cu") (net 4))
 (segment (start 172.663 102.613) (end 172.663 98.213) (width 1) (layer "B.Cu") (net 4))
 (segment (start 168.663 88.1) (end 168.663 86.35) (width 1) (layer "B.Cu") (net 4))
 (segment (start 164.805 102.85) (end 165.055 103.1) (width 1) (layer "B.Cu") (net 4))
 (segment (start 165.055 91.708) (end 168.663 88.1) (width 1) (layer "B.Cu") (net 4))
 (segment (start 168.663 84.35) (end 170.068 82.945) (width 1) (layer "B.Cu") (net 4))
 (segment (start 143.055 106.35) (end 144.68 104.725) (width 1) (layer "B.Cu") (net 4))
 (segment (start 164.305 113.85) (end 164.305 113.3025) (width 1) (layer "B.Cu") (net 4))
 (segment (start 152.393 98.25) (end 151.163 99.48) (width 1) (layer "B.Cu") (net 4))
 (segment (start 137.805 106.35) (end 137.755 106.3) (width 1) (layer "B.Cu") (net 4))
 (segment (start 170.3 95.85) (end 165.055 95.85) (width 1) (layer "B.Cu") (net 4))
 (segment (start 151.163 99.48) (end 151.163 100.708) (width 1) (layer "B.Cu") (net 4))
 (segment (start 134.755 105.43) (end 134.755 101.6) (width 1) (layer "B.Cu") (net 4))
 (segment (start 137.755 106.3) (end 135.625 106.3) (width 1) (layer "B.Cu") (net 4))
 (segment (start 146.305 103.1) (end 145.105 104.3) (width 1) (layer "B.Cu") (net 4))
 (segment (start 153.305 102.85) (end 164.805 102.85) (width 1) (layer "B.Cu") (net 4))
 (segment (start 168.31 116.39) (end 169.515 116.39) (width 1) (layer "B.Cu") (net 11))
 (segment (start 171.162 114.957) (end 174.663 114.957) (width 1) (layer "B.Cu") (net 11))
 (segment (start 171.055 114.85) (end 171.055 105.6) (width 1) (layer "B.Cu") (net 11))
 (segment (start 164.305 117.8025) (end 167.3225 117.8025) (width 1) (layer "B.Cu") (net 11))
 (segment (start 168.31 116.815) (end 168.31 116.39) (width 1) (layer "B.Cu") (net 11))
 (segment (start 169.515 116.39) (end 171.055 114.85) (width 1) (layer "B.Cu") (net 11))
 (segment (start 171.055 114.85) (end 171.162 114.957) (width 1) (layer "B.Cu") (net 11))
 (segment (start 167.3225 117.8025) (end 168.31 116.815) (width 1) (layer "B.Cu") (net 11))
 (segment (start 171.055 105.6) (end 168.555 103.1) (width 1) (layer "B.Cu") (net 11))
 (segment (start 165.163 87.812) (end 165.163 86.35) (width 1) (layer "B.Cu") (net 2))
 (segment (start 142.088 87.175) (end 142.913 86.35) (width 1) (layer "B.Cu") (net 2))
 (segment (start 165.913 79.4525) (end 165.913 75.067) (width 1) (layer "B.Cu") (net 2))
 (segment (start 142.913 86.35) (end 146.413 86.35) (width 1) (layer "B.Cu") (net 2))
 (segment (start 165.6155 79.85) (end 165.5655 79.8) (width 1) (layer "B.Cu") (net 2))
 (segment (start 165.913 75.067) (end 165.878 75.032) (width 1) (layer "B.Cu") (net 2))
 (segment (start 165.163 84.1) (end 165.913 83.35) (width 1) (layer "B.Cu") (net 2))
 (segment (start 165.913 83.35) (end 165.913 80.1475) (width 1) (layer "B.Cu") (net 2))
 (segment (start 133.018 91.995) (end 137.863 87.15) (width 1) (layer "B.Cu") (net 2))
 (segment (start 174.663 74.1) (end 172.913 72.35) (width 1) (layer "B.Cu") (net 2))
 (segment (start 158.55 94.425) (end 165.163 87.812) (width 1) (layer "B.Cu") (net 2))
 (segment (start 168.163 79.85) (end 165.6155 79.85) (width 1) (layer "B.Cu") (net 2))
 (segment (start 146.413 89.1) (end 146.413 86.35) (width 1) (layer "B.Cu") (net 2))
 (segment (start 137.863 87.15) (end 137.888 87.175) (width 1) (layer "B.Cu") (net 2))
 (segment (start 137.863 81.925) (end 136.25 81.925) (width 1) (layer "B.Cu") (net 2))
 (segment (start 165.163 86.35) (end 165.163 84.1) (width 1) (layer "B.Cu") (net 2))
 (segment (start 174.663 76.465) (end 174.663 74.1) (width 1) (layer "B.Cu") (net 2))
 (segment (start 130.521 91.995) (end 133.018 91.995) (width 1) (layer "B.Cu") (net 2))
 (segment (start 165.913 80.1475) (end 165.5655 79.8) (width 1) (layer "B.Cu") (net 2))
 (segment (start 172.913 72.35) (end 166.913 72.35) (width 1) (layer "B.Cu") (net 2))
 (segment (start 165.5655 79.8) (end 165.913 79.4525) (width 1) (layer "B.Cu") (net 2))
 (segment (start 165.878 73.385) (end 165.878 75.032) (width 1) (layer "B.Cu") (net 2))
 (segment (start 166.913 72.35) (end 165.878 73.385) (width 1) (layer "B.Cu") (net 2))
 (segment (start 153.575 94.425) (end 158.55 94.425) (width 1) (layer "B.Cu") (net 2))
 (segment (start 152.393 91.1) (end 152.393 93.243) (width 1) (layer "B.Cu") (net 2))
 (segment (start 137.863 87.15) (end 137.863 81.925) (width 1) (layer "B.Cu") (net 2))
 (segment (start 136.25 81.925) (end 134.863 80.538) (width 1) (layer "B.Cu") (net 2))
 (segment (start 148.413 91.1) (end 146.413 89.1) (width 1) (layer "B.Cu") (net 2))
 (segment (start 152.393 91.1) (end 148.413 91.1) (width 1) (layer "B.Cu") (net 2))
 (segment (start 137.888 87.175) (end 142.088 87.175) (width 1) (layer "B.Cu") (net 2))
 (segment (start 152.393 93.243) (end 153.575 94.425) (width 1) (layer "B.Cu") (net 2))
 (segment (start 134.863 80.538) (end 134.863 77.225) (width 1) (layer "B.Cu") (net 2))
 (segment (start 155.163 83.207) (end 155.195 83.175) (width 1) (layer "B.Cu") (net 5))
 (segment (start 149.738 83.175) (end 149.738 86.175) (width 1) (layer "B.Cu") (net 5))
 (segment (start 149.738 83.175) (end 155.195 83.175) (width 1) (layer "B.Cu") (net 5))
 (segment (start 146.363 79.8) (end 149.738 83.175) (width 1) (layer "B.Cu") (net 5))
 (segment (start 163.6605 79.8) (end 161.11525 77.25475) (width 1) (layer "B.Cu") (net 5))
 (segment (start 149.738 86.175) (end 149.913 86.35) (width 1) (layer "B.Cu") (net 5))
 (segment (start 155.163 85.1475) (end 155.163 83.207) (width 1) (layer "B.Cu") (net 5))
 (segment (start 161.11525 77.25475) (end 163.338 75.032) (width 1) (layer "B.Cu") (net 5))
 (segment (start 155.195 83.175) (end 163.338 75.032) (width 1) (layer "B.Cu") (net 5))
 (segment (start 146.363 76.119) (end 146.363 79.8) (width 1) (layer "B.Cu") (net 5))
 (segment (start 177.663 112.588) (end 177.663 107.195) (width 1) (layer "B.Cu") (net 13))
 (segment (start 179.163 114.088) (end 177.663 112.588) (width 1) (layer "B.Cu") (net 13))
 (segment (start 179.163 114.957) (end 179.163 114.088) (width 1) (layer "B.Cu") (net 13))
 (segment (start 177.663 107.195) (end 177.608 107.14) (width 1) (layer "B.Cu") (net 13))
 (segment (start 177.608 102.06) (end 177.608 79.217) (width 1) (layer "B.Cu") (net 12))
 (segment (start 179.163 77.662) (end 179.163 76.465) (width 1) (layer "B.Cu") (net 12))
 (segment (start 177.608 79.217) (end 179.163 77.662) (width 1) (layer "B.Cu") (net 12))
 (segment (start 130.413 111.255) (end 130.413 99.887) (width 1) (layer "B.Cu") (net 3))
 (segment (start 127.9 111.255) (end 126.555 112.6) (width 1) (layer "B.Cu") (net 3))
 (segment (start 150.955 118.345) (end 150.955 115.248) (width 1) (layer "B.Cu") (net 3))
 (segment (start 126.555 112.6) (end 126.555 118.35) (width 1) (layer "B.Cu") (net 3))
 (segment (start 140.755 99.455) (end 140.755 101.6) (width 1) (layer "B.Cu") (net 3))
 (segment (start 132.2 98.1) (end 139.4 98.1) (width 1) (layer "B.Cu") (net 3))
 (segment (start 149.2 120.1) (end 150.955 118.345) (width 1) (layer "B.Cu") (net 3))
 (segment (start 128.305 120.1) (end 149.2 120.1) (width 1) (layer "B.Cu") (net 3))
 (segment (start 130.413 111.255) (end 127.9 111.255) (width 1) (layer "B.Cu") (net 3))
 (segment (start 139.4 98.1) (end 140.755 99.455) (width 1) (layer "B.Cu") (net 3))
 (segment (start 130.413 99.887) (end 132.2 98.1) (width 1) (layer "B.Cu") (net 3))
 (segment (start 126.555 118.35) (end 128.305 120.1) (width 1) (layer "B.Cu") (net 3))
 (segment (start 141.613 72.35) (end 149.3 72.35) (width 1) (layer "B.Cu") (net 6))
 (segment (start 151.063 74.113) (end 151.063 76.119) (width 1) (layer "B.Cu") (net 6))
 (segment (start 140.663 72.35) (end 141.613 72.35) (width 1) (layer "B.Cu") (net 6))
 (segment (start 140.863 77.225) (end 140.863 72.55) (width 1) (layer "B.Cu") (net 6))
 (segment (start 130.521 86.915) (end 130.521 75.992) (width 1) (layer "B.Cu") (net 6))
 (segment (start 149.3 72.35) (end 151.063 74.113) (width 1) (layer "B.Cu") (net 6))
 (segment (start 140.863 72.55) (end 140.663 72.35) (width 1) (layer "B.Cu") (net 6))
 (segment (start 134.163 72.35) (end 141.613 72.35) (width 1) (layer "B.Cu") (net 6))
 (segment (start 130.521 75.992) (end 134.163 72.35) (width 1) (layer "B.Cu") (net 6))
 (segment (start 155.8855 97.2975) (end 157 97.2975) (width 1) (layer "B.Cu") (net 9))
 (segment (start 154.933 98.25) (end 155.8855 97.2975) (width 1) (layer "B.Cu") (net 9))
 (segment (start 154.933 87.2825) (end 155.163 87.0525) (width 1) (layer "B.Cu") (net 1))
 (segment (start 154.933 91.1) (end 154.933 87.2825) (width 1) (layer "B.Cu") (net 1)))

